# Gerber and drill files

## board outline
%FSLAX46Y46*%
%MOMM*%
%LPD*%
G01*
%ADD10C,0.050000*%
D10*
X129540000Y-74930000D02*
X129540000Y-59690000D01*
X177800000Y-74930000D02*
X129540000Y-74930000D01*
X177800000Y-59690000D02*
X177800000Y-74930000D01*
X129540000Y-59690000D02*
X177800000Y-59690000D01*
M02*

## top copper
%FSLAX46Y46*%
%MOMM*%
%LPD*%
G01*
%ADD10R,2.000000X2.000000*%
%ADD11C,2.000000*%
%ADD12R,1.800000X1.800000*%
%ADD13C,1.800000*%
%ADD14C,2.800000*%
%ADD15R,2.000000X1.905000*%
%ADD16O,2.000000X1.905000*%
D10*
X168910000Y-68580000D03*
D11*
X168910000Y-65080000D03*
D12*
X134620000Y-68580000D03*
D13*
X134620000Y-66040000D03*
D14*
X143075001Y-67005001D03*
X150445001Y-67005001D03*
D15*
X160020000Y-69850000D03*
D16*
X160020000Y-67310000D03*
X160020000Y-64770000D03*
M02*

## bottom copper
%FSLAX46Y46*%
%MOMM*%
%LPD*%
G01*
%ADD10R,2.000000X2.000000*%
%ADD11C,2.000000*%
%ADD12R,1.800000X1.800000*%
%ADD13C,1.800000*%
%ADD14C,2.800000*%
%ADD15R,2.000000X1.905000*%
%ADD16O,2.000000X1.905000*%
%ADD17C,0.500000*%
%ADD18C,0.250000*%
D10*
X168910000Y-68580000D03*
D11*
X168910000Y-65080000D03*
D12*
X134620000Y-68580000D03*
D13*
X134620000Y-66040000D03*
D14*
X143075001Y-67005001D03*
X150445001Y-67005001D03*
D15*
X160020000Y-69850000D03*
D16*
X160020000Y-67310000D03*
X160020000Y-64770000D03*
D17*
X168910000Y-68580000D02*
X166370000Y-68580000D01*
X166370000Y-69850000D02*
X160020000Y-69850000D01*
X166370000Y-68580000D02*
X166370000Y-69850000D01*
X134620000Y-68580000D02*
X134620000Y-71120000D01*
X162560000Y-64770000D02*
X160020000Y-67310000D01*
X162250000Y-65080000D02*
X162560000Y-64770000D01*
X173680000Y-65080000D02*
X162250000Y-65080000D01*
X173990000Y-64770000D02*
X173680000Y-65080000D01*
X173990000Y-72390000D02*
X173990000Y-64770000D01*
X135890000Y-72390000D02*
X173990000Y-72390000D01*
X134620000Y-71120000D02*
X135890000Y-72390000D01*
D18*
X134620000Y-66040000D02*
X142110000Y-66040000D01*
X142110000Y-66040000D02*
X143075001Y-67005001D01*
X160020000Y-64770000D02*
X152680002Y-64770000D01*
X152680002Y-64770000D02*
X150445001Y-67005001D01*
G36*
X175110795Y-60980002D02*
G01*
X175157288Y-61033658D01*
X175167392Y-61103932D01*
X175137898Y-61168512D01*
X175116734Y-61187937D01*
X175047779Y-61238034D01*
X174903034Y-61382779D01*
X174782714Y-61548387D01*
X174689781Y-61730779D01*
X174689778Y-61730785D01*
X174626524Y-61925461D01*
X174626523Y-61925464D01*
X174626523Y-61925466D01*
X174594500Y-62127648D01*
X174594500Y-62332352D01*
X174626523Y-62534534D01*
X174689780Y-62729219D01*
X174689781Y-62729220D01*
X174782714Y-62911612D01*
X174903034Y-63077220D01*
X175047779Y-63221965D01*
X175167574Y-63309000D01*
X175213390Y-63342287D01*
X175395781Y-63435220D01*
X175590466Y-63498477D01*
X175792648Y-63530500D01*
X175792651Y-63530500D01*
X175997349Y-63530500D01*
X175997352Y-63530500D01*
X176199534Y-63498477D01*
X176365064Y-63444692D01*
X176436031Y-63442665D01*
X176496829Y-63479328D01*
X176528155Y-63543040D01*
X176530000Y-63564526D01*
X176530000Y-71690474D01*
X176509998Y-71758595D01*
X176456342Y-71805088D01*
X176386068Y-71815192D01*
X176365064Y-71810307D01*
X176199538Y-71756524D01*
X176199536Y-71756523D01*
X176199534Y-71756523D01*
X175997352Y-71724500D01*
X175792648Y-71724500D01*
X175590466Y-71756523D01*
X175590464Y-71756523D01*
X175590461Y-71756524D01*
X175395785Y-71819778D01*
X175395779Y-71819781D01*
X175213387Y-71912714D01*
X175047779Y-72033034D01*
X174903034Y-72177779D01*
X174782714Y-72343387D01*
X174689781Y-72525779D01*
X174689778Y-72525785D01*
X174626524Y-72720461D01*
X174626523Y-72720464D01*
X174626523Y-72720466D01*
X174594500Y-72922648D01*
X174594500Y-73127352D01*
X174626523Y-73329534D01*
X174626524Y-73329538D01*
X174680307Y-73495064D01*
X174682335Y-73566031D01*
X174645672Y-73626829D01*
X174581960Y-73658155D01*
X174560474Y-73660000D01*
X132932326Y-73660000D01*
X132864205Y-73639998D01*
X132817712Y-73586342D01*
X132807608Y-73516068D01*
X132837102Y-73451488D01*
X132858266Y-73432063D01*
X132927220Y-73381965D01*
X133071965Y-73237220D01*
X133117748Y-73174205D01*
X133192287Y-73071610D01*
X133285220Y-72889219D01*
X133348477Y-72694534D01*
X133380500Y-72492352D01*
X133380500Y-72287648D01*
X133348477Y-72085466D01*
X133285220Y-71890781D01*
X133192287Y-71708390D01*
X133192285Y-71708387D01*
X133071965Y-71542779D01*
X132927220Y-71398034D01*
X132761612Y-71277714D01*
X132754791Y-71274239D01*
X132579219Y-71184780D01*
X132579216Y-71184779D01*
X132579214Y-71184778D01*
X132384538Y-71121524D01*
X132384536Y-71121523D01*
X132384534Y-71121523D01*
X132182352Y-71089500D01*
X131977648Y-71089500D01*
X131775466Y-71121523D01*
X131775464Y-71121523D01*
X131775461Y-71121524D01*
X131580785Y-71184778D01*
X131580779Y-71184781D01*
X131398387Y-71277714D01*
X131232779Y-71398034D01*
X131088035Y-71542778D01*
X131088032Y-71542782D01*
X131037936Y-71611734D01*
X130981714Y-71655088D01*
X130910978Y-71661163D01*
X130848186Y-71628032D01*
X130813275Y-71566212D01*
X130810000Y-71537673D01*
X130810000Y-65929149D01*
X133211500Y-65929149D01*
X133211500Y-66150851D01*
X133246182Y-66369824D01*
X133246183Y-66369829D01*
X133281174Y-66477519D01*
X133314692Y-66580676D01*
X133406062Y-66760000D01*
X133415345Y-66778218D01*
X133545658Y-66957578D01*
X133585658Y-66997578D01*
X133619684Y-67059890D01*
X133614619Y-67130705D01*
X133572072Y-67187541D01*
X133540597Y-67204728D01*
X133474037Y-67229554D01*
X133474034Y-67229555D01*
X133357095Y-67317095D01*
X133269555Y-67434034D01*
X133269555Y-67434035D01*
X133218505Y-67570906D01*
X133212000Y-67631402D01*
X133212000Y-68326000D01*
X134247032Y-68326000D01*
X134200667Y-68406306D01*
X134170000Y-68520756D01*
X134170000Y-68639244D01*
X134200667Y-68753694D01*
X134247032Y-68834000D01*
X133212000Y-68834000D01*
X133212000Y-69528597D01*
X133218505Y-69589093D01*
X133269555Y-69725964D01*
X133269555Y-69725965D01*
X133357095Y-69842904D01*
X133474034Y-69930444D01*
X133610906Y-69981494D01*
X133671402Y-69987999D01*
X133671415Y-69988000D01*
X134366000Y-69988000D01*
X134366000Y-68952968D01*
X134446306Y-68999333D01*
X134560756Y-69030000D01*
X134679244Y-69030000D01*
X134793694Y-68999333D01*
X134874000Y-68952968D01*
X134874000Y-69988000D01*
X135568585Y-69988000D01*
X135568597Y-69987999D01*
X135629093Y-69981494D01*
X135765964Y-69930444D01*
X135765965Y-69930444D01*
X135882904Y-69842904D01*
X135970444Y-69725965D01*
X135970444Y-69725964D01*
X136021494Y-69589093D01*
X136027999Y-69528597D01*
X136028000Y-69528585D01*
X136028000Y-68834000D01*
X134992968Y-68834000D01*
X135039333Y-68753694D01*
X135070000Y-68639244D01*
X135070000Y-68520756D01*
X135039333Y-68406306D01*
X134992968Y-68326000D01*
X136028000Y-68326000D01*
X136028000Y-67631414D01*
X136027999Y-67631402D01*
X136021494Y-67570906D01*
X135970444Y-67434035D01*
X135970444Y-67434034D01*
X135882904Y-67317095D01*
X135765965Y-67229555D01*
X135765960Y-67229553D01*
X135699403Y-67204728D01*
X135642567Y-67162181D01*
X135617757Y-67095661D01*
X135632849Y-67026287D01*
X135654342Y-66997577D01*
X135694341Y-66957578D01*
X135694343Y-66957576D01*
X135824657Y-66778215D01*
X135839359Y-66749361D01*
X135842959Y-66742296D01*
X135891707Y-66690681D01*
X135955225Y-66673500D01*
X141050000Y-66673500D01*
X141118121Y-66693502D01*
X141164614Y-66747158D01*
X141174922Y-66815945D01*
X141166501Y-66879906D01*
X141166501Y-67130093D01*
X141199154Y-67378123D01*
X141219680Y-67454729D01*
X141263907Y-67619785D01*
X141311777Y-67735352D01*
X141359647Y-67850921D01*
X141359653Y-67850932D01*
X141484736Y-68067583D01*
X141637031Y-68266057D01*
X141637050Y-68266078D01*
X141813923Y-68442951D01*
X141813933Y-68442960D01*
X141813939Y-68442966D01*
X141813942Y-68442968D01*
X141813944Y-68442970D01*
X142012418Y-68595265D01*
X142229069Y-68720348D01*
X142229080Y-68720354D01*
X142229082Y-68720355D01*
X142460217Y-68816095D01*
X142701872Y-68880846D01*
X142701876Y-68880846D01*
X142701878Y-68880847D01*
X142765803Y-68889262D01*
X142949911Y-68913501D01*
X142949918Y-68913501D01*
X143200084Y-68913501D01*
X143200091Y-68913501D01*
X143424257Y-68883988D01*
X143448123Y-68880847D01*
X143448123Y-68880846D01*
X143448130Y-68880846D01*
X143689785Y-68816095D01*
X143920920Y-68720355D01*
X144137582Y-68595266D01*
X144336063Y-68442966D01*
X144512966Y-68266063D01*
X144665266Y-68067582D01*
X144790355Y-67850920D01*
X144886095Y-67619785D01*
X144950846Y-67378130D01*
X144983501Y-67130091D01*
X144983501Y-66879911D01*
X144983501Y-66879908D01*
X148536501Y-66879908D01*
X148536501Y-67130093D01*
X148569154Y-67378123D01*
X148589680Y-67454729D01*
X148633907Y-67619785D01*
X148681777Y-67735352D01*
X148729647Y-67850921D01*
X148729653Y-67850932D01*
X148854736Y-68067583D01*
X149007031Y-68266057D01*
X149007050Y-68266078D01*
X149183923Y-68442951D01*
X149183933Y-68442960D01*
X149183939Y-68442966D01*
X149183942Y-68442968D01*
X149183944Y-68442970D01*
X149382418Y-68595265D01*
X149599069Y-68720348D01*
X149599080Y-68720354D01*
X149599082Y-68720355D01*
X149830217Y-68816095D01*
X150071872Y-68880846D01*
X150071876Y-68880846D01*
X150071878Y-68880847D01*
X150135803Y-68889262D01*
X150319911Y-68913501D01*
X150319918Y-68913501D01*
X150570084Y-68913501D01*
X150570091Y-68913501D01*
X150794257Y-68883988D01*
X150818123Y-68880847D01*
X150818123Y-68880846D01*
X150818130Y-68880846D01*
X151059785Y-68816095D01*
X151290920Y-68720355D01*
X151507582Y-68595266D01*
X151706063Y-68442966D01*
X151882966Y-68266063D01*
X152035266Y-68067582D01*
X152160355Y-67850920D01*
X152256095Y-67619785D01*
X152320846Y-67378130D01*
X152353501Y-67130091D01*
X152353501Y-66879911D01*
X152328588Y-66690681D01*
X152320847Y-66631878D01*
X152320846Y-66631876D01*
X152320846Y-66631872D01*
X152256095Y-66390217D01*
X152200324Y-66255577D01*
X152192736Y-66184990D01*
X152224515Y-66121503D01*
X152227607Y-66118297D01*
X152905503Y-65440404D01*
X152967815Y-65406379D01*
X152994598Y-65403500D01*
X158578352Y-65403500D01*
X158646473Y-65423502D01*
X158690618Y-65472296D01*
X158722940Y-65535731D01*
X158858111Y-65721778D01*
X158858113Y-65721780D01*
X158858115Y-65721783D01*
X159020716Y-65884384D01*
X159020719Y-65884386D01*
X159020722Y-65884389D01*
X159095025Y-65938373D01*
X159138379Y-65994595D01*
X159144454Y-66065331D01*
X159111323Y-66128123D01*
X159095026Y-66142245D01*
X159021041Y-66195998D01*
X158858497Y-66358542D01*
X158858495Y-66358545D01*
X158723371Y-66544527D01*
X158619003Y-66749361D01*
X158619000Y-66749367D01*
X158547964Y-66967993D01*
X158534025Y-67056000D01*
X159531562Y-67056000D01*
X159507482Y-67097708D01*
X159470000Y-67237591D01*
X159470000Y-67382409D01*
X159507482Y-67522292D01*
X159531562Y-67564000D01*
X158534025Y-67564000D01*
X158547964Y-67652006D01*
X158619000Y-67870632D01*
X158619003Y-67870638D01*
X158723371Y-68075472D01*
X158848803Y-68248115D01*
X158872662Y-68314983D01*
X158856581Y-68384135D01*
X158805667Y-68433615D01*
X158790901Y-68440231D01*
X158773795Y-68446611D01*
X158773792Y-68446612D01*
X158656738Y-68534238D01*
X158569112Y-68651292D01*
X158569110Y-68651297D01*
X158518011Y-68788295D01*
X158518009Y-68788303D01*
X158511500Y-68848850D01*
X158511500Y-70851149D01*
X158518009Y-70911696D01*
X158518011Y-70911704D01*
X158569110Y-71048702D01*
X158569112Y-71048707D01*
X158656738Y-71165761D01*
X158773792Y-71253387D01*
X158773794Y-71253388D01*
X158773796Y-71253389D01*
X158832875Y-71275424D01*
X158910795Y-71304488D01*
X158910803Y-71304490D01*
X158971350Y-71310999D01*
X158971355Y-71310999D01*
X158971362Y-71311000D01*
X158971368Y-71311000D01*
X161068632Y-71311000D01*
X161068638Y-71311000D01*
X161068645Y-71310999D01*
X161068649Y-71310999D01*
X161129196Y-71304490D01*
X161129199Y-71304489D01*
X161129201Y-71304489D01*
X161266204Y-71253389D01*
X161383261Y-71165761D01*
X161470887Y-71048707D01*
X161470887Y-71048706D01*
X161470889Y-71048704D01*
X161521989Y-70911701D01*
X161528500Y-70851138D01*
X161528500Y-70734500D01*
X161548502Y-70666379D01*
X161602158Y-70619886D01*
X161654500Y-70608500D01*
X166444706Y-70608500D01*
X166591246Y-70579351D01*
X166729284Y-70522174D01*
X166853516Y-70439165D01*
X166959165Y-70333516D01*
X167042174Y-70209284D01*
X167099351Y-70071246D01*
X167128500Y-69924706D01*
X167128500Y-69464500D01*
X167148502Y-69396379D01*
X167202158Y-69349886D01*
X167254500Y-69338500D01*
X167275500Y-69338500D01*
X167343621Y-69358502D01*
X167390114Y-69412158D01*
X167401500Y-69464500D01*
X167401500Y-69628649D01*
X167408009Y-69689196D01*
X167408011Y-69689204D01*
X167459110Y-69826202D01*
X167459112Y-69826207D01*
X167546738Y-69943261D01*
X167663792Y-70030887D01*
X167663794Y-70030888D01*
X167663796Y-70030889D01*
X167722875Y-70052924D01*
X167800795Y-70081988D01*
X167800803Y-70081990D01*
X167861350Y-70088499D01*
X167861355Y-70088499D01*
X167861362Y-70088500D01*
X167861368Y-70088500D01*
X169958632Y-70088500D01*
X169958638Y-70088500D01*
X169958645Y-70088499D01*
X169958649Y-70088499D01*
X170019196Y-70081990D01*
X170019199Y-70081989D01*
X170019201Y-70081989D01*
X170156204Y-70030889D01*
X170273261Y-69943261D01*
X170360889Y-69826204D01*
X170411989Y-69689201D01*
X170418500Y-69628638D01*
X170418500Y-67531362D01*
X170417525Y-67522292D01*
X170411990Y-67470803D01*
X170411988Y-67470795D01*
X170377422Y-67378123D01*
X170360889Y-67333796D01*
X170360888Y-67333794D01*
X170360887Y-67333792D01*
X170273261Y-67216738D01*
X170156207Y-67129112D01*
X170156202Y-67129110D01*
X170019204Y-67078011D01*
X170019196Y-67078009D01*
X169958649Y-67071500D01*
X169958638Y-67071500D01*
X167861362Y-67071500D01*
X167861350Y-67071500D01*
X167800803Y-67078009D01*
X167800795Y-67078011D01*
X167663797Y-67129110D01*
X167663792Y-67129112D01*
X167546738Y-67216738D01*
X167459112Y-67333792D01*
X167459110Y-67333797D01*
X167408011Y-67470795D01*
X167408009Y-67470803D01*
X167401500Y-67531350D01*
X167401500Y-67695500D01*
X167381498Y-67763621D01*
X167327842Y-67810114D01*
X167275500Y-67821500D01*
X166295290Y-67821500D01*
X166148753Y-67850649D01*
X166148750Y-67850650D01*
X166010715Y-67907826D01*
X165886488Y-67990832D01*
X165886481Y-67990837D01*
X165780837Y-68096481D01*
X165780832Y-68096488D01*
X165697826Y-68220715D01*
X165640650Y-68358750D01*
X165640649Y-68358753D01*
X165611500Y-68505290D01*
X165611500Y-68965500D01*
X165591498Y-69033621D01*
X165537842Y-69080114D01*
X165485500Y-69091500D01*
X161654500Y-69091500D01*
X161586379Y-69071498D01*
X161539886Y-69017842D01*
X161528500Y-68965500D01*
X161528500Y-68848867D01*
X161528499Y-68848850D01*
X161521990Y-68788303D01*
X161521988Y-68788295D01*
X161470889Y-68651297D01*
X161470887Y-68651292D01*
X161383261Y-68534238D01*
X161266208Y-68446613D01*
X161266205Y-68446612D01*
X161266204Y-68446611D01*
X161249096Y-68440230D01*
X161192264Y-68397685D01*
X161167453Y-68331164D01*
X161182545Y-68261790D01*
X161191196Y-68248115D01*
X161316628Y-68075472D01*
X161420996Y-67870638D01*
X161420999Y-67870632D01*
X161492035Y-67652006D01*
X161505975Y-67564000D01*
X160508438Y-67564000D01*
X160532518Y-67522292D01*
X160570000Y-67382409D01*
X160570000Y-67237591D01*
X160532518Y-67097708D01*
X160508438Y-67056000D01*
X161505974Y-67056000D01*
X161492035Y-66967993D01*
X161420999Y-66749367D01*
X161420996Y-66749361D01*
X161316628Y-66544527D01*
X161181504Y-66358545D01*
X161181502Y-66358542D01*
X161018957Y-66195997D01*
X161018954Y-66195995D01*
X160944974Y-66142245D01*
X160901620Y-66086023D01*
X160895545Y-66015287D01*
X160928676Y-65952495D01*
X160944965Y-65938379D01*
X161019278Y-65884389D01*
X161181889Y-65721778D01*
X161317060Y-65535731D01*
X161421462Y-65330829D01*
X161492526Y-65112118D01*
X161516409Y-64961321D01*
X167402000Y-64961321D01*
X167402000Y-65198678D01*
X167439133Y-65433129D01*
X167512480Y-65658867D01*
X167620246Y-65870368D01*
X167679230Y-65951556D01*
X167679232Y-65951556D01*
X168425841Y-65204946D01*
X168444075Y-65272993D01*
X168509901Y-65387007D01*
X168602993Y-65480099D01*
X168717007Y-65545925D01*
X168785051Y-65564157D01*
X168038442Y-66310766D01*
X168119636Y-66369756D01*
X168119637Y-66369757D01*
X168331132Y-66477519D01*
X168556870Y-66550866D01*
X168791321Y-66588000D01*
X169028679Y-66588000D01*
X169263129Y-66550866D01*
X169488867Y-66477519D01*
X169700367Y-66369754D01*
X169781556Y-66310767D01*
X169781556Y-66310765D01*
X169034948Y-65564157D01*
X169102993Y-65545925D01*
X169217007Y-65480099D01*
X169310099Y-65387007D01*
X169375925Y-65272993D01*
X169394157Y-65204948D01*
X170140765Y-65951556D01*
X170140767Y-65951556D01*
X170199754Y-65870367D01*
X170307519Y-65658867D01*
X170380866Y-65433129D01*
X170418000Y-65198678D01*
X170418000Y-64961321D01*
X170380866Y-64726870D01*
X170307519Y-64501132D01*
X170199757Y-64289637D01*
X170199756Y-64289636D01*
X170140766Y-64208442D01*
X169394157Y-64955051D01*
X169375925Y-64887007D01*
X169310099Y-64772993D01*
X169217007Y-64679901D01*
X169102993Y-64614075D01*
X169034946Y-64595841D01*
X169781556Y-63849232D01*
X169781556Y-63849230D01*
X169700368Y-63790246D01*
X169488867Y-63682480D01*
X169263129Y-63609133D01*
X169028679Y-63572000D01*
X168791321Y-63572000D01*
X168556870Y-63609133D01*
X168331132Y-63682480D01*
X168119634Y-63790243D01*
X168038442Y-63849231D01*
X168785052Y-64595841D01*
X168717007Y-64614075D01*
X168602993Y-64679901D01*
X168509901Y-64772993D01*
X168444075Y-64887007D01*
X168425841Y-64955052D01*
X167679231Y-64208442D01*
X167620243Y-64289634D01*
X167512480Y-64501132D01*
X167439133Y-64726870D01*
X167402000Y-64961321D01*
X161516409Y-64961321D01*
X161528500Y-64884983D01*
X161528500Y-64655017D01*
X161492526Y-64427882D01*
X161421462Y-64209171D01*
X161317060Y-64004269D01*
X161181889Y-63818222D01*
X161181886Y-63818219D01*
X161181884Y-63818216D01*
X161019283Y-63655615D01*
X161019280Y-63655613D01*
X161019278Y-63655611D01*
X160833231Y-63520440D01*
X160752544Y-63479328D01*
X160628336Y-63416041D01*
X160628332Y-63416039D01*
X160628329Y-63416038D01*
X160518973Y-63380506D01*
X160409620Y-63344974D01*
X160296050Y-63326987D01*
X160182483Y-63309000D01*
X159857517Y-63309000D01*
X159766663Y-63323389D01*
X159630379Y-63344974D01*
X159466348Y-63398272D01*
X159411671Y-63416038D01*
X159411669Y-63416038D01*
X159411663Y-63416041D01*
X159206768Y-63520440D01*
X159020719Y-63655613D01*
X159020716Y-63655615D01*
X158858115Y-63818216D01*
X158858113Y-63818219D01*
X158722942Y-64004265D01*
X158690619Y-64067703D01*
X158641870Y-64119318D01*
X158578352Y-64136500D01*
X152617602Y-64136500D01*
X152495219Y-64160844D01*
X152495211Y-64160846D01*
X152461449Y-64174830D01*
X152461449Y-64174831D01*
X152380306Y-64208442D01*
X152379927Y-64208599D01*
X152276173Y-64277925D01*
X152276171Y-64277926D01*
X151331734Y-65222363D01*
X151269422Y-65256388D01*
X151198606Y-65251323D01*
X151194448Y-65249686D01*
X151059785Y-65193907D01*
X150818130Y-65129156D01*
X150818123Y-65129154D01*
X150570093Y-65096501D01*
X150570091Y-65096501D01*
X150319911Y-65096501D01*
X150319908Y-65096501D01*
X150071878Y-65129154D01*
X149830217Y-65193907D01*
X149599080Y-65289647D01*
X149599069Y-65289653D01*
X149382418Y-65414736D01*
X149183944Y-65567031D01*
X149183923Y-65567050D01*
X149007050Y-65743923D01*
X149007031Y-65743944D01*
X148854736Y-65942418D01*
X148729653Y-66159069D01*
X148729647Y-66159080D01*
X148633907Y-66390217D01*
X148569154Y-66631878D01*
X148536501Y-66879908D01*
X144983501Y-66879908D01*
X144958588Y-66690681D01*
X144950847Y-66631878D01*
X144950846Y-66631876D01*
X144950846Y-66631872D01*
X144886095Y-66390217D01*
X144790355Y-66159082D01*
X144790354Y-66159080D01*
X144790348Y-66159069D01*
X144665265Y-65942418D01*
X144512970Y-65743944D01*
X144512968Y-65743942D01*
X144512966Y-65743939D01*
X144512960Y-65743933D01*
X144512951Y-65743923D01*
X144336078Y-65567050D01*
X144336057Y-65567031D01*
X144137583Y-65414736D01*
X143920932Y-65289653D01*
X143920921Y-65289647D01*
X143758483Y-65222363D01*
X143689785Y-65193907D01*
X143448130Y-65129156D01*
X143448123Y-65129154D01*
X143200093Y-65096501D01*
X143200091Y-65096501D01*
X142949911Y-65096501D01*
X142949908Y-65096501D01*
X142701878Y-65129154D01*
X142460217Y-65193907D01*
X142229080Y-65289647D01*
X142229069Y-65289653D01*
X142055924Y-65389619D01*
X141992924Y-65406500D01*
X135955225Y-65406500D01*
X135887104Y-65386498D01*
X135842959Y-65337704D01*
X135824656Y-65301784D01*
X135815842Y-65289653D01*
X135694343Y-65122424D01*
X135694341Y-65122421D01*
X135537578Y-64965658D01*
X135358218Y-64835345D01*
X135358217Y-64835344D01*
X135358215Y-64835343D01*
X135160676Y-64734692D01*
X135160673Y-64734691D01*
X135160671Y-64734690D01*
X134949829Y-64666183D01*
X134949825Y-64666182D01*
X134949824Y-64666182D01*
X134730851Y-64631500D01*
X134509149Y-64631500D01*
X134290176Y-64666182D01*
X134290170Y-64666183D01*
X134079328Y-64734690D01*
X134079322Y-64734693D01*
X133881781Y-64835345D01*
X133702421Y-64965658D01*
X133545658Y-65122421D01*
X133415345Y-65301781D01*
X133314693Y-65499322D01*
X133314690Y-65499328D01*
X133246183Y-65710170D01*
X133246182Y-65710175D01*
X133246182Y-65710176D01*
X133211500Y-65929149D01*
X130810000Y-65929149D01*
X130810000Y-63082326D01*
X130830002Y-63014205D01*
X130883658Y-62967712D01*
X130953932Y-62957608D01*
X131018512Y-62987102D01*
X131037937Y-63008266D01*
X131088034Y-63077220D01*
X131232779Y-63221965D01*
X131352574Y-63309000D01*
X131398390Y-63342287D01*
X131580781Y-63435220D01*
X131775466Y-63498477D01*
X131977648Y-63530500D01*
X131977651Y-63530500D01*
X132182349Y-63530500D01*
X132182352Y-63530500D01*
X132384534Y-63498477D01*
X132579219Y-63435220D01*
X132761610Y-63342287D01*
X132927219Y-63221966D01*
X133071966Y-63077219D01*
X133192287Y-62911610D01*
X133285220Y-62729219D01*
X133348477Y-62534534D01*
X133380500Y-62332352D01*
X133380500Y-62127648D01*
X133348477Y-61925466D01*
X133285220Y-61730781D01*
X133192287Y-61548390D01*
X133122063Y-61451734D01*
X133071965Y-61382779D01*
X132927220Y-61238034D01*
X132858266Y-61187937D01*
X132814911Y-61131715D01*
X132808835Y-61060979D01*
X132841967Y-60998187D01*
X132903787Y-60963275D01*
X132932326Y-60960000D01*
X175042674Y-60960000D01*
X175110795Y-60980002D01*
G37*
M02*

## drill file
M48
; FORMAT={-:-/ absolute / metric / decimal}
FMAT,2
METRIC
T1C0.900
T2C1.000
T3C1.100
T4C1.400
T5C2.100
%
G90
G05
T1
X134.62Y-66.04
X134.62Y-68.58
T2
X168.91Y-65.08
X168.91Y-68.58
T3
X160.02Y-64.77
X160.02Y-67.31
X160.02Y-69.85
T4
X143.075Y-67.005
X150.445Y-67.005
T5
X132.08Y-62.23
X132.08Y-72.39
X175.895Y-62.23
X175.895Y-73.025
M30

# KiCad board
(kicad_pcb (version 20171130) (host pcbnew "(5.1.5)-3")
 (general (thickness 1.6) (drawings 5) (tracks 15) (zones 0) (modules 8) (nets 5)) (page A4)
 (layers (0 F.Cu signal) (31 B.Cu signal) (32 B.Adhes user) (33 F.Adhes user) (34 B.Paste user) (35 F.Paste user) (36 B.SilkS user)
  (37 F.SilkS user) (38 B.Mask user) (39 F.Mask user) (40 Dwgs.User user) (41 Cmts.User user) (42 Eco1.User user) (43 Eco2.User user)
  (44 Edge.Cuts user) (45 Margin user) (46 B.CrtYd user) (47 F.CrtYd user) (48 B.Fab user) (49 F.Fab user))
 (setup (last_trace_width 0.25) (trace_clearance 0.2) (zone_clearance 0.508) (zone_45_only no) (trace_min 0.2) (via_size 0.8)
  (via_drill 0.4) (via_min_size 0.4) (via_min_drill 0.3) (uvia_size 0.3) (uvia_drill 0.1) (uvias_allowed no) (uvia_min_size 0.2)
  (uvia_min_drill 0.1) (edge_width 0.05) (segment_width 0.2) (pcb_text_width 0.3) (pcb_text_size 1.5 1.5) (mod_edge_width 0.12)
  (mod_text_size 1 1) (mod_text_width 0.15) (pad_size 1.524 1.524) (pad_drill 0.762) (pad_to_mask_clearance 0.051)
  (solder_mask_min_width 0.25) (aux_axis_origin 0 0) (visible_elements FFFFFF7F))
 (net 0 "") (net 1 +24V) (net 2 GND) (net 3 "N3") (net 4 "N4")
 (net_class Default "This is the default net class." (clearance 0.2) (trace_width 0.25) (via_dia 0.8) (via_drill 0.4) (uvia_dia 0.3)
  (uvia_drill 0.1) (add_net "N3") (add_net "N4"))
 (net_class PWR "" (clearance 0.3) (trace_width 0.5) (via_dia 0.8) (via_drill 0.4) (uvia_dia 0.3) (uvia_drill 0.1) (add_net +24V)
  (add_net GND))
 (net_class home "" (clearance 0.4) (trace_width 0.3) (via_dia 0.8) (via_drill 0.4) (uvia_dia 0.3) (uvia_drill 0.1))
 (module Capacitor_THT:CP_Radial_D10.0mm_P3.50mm (layer F.Cu) (at 168.91 68.58 90)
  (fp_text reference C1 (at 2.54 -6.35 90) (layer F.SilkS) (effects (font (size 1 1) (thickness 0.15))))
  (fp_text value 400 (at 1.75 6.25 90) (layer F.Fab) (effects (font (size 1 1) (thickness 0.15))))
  (pad 1 thru_hole rect (at 0 0 90) (size 2 2) (drill 1) (layers *.Cu *.Mask) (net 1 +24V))
  (pad 2 thru_hole circle (at 3.5 0 90) (size 2 2) (drill 1) (layers *.Cu *.Mask) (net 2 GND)))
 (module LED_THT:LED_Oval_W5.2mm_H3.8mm (layer F.Cu) (at 134.62 68.58 90)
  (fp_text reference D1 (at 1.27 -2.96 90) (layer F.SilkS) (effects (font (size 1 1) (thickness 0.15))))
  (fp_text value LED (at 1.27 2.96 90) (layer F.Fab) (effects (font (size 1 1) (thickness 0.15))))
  (pad 1 thru_hole rect (at 0 0 90) (size 1.8 1.8) (drill 0.9) (layers *.Cu *.Mask) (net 2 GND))
  (pad 2 thru_hole circle (at 2.54 0 90) (size 1.8 1.8) (drill 0.9) (layers *.Cu *.Mask) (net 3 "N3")))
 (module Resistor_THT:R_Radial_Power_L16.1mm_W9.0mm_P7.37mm (layer F.Cu) (at 143.075001 67.005001)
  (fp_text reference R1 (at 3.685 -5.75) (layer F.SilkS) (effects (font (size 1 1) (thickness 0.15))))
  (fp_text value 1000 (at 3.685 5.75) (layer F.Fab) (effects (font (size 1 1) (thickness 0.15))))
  (pad 1 thru_hole circle (at 0 0) (size 2.8 2.8) (drill 1.4) (layers *.Cu *.Mask) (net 3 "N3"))
  (pad 2 thru_hole circle (at 7.37 0) (size 2.8 2.8) (drill 1.4) (layers *.Cu *.Mask) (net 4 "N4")))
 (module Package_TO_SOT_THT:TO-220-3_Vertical (layer F.Cu) (at 160.02 69.85 90)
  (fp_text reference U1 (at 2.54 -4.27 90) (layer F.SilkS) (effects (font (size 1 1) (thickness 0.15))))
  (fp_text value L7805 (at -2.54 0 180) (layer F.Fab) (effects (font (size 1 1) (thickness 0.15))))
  (pad 1 thru_hole rect (at 0 0 90) (size 1.905 2) (drill 1.1) (layers *.Cu *.Mask) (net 1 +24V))
  (pad 2 thru_hole oval (at 2.54 0 90) (size 1.905 2) (drill 1.1) (layers *.Cu *.Mask) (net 2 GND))
  (pad 3 thru_hole oval (at 5.08 0 90) (size 1.905 2) (drill 1.1) (layers *.Cu *.Mask) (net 4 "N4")))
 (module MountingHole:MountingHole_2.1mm (layer F.Cu) (at 132.08 62.23)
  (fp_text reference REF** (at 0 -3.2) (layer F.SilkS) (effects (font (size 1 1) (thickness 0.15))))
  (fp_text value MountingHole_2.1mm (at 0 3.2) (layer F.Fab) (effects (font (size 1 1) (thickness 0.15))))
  (pad "" np_thru_hole circle (at 0 0) (size 2.1 2.1) (drill 2.1) (layers *.Cu *.Mask)))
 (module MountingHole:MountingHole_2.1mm (layer F.Cu) (at 175.895 62.23)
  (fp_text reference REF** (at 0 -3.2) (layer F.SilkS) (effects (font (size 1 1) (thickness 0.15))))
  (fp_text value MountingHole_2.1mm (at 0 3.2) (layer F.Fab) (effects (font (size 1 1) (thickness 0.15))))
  (pad "" np_thru_hole circle (at 0 0) (size 2.1 2.1) (drill 2.1) (layers *.Cu *.Mask)))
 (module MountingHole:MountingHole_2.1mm (layer F.Cu) (at 175.895 73.025)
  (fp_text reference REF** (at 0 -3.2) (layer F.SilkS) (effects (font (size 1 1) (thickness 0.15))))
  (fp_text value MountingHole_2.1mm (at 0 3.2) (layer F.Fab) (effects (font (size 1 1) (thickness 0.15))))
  (pad "" np_thru_hole circle (at 0 0) (size 2.1 2.1) (drill 2.1) (layers *.Cu *.Mask)))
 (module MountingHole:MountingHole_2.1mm (layer F.Cu) (at 132.08 72.39)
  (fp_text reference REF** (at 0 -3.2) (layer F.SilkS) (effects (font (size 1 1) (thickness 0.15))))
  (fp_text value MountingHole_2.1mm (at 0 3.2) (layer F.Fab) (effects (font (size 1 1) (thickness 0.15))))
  (pad "" np_thru_hole circle (at 0 0) (size 2.1 2.1) (drill 2.1) (layers *.Cu *.Mask)))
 (gr_line (start 129.54 74.93) (end 129.54 59.69) (layer Edge.Cuts) (width 0.05))
 (gr_line (start 177.8 74.93) (end 129.54 74.93) (layer Edge.Cuts) (width 0.05))
 (gr_line (start 177.8 59.69) (end 177.8 74.93) (layer Edge.Cuts) (width 0.05))
 (gr_line (start 129.54 59.69) (end 177.8 59.69) (layer Edge.Cuts) (width 0.05))
 (segment (start 168.91 68.58) (end 166.37 68.58) (width 0.5) (layer B.Cu) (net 1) (status 400000))
 (segment (start 166.37 69.85) (end 160.02 69.85) (width 0.5) (layer B.Cu) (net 1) (status 800000))
 (segment (start 166.37 68.58) (end 166.37 69.85) (width 0.5) (layer B.Cu) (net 1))
 (segment (start 134.62 68.58) (end 134.62 71.12) (width 0.5) (layer B.Cu) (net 2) (status 400000))
 (segment (start 162.56 64.77) (end 160.02 67.31) (width 0.5) (layer B.Cu) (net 2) (status 800000))
 (segment (start 162.25 65.08) (end 162.56 64.77) (width 0.5) (layer B.Cu) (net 2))
 (segment (start 173.68 65.08) (end 162.25 65.08) (width 0.5) (layer B.Cu) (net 2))
 (segment (start 173.99 64.77) (end 173.68 65.08) (width 0.5) (layer B.Cu) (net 2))
 (segment (start 173.99 72.39) (end 173.99 64.77) (width 0.5) (layer B.Cu) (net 2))
 (segment (start 135.89 72.39) (end 173.99 72.39) (width 0.5) (layer B.Cu) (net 2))
 (segment (start 134.62 71.12) (end 135.89 72.39) (width 0.5) (layer B.Cu) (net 2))
 (segment (start 134.62 66.04) (end 142.11 66.04) (width 0.25) (layer B.Cu) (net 3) (status C00000))
 (segment (start 142.11 66.04) (end 143.075001 67.005001) (width 0.25) (layer B.Cu) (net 3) (status C00000))
 (segment (start 160.02 64.77) (end 152.680002 64.77) (width 0.25) (layer B.Cu) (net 4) (status 400000))
 (segment (start 152.680002 64.77) (end 150.445001 67.005001) (width 0.25) (layer B.Cu) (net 4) (status 800000))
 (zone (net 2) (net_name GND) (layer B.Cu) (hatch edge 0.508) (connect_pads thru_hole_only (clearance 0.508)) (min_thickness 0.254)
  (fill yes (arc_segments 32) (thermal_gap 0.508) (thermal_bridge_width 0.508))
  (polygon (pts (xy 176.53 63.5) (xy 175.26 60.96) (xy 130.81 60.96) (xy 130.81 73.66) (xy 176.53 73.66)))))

